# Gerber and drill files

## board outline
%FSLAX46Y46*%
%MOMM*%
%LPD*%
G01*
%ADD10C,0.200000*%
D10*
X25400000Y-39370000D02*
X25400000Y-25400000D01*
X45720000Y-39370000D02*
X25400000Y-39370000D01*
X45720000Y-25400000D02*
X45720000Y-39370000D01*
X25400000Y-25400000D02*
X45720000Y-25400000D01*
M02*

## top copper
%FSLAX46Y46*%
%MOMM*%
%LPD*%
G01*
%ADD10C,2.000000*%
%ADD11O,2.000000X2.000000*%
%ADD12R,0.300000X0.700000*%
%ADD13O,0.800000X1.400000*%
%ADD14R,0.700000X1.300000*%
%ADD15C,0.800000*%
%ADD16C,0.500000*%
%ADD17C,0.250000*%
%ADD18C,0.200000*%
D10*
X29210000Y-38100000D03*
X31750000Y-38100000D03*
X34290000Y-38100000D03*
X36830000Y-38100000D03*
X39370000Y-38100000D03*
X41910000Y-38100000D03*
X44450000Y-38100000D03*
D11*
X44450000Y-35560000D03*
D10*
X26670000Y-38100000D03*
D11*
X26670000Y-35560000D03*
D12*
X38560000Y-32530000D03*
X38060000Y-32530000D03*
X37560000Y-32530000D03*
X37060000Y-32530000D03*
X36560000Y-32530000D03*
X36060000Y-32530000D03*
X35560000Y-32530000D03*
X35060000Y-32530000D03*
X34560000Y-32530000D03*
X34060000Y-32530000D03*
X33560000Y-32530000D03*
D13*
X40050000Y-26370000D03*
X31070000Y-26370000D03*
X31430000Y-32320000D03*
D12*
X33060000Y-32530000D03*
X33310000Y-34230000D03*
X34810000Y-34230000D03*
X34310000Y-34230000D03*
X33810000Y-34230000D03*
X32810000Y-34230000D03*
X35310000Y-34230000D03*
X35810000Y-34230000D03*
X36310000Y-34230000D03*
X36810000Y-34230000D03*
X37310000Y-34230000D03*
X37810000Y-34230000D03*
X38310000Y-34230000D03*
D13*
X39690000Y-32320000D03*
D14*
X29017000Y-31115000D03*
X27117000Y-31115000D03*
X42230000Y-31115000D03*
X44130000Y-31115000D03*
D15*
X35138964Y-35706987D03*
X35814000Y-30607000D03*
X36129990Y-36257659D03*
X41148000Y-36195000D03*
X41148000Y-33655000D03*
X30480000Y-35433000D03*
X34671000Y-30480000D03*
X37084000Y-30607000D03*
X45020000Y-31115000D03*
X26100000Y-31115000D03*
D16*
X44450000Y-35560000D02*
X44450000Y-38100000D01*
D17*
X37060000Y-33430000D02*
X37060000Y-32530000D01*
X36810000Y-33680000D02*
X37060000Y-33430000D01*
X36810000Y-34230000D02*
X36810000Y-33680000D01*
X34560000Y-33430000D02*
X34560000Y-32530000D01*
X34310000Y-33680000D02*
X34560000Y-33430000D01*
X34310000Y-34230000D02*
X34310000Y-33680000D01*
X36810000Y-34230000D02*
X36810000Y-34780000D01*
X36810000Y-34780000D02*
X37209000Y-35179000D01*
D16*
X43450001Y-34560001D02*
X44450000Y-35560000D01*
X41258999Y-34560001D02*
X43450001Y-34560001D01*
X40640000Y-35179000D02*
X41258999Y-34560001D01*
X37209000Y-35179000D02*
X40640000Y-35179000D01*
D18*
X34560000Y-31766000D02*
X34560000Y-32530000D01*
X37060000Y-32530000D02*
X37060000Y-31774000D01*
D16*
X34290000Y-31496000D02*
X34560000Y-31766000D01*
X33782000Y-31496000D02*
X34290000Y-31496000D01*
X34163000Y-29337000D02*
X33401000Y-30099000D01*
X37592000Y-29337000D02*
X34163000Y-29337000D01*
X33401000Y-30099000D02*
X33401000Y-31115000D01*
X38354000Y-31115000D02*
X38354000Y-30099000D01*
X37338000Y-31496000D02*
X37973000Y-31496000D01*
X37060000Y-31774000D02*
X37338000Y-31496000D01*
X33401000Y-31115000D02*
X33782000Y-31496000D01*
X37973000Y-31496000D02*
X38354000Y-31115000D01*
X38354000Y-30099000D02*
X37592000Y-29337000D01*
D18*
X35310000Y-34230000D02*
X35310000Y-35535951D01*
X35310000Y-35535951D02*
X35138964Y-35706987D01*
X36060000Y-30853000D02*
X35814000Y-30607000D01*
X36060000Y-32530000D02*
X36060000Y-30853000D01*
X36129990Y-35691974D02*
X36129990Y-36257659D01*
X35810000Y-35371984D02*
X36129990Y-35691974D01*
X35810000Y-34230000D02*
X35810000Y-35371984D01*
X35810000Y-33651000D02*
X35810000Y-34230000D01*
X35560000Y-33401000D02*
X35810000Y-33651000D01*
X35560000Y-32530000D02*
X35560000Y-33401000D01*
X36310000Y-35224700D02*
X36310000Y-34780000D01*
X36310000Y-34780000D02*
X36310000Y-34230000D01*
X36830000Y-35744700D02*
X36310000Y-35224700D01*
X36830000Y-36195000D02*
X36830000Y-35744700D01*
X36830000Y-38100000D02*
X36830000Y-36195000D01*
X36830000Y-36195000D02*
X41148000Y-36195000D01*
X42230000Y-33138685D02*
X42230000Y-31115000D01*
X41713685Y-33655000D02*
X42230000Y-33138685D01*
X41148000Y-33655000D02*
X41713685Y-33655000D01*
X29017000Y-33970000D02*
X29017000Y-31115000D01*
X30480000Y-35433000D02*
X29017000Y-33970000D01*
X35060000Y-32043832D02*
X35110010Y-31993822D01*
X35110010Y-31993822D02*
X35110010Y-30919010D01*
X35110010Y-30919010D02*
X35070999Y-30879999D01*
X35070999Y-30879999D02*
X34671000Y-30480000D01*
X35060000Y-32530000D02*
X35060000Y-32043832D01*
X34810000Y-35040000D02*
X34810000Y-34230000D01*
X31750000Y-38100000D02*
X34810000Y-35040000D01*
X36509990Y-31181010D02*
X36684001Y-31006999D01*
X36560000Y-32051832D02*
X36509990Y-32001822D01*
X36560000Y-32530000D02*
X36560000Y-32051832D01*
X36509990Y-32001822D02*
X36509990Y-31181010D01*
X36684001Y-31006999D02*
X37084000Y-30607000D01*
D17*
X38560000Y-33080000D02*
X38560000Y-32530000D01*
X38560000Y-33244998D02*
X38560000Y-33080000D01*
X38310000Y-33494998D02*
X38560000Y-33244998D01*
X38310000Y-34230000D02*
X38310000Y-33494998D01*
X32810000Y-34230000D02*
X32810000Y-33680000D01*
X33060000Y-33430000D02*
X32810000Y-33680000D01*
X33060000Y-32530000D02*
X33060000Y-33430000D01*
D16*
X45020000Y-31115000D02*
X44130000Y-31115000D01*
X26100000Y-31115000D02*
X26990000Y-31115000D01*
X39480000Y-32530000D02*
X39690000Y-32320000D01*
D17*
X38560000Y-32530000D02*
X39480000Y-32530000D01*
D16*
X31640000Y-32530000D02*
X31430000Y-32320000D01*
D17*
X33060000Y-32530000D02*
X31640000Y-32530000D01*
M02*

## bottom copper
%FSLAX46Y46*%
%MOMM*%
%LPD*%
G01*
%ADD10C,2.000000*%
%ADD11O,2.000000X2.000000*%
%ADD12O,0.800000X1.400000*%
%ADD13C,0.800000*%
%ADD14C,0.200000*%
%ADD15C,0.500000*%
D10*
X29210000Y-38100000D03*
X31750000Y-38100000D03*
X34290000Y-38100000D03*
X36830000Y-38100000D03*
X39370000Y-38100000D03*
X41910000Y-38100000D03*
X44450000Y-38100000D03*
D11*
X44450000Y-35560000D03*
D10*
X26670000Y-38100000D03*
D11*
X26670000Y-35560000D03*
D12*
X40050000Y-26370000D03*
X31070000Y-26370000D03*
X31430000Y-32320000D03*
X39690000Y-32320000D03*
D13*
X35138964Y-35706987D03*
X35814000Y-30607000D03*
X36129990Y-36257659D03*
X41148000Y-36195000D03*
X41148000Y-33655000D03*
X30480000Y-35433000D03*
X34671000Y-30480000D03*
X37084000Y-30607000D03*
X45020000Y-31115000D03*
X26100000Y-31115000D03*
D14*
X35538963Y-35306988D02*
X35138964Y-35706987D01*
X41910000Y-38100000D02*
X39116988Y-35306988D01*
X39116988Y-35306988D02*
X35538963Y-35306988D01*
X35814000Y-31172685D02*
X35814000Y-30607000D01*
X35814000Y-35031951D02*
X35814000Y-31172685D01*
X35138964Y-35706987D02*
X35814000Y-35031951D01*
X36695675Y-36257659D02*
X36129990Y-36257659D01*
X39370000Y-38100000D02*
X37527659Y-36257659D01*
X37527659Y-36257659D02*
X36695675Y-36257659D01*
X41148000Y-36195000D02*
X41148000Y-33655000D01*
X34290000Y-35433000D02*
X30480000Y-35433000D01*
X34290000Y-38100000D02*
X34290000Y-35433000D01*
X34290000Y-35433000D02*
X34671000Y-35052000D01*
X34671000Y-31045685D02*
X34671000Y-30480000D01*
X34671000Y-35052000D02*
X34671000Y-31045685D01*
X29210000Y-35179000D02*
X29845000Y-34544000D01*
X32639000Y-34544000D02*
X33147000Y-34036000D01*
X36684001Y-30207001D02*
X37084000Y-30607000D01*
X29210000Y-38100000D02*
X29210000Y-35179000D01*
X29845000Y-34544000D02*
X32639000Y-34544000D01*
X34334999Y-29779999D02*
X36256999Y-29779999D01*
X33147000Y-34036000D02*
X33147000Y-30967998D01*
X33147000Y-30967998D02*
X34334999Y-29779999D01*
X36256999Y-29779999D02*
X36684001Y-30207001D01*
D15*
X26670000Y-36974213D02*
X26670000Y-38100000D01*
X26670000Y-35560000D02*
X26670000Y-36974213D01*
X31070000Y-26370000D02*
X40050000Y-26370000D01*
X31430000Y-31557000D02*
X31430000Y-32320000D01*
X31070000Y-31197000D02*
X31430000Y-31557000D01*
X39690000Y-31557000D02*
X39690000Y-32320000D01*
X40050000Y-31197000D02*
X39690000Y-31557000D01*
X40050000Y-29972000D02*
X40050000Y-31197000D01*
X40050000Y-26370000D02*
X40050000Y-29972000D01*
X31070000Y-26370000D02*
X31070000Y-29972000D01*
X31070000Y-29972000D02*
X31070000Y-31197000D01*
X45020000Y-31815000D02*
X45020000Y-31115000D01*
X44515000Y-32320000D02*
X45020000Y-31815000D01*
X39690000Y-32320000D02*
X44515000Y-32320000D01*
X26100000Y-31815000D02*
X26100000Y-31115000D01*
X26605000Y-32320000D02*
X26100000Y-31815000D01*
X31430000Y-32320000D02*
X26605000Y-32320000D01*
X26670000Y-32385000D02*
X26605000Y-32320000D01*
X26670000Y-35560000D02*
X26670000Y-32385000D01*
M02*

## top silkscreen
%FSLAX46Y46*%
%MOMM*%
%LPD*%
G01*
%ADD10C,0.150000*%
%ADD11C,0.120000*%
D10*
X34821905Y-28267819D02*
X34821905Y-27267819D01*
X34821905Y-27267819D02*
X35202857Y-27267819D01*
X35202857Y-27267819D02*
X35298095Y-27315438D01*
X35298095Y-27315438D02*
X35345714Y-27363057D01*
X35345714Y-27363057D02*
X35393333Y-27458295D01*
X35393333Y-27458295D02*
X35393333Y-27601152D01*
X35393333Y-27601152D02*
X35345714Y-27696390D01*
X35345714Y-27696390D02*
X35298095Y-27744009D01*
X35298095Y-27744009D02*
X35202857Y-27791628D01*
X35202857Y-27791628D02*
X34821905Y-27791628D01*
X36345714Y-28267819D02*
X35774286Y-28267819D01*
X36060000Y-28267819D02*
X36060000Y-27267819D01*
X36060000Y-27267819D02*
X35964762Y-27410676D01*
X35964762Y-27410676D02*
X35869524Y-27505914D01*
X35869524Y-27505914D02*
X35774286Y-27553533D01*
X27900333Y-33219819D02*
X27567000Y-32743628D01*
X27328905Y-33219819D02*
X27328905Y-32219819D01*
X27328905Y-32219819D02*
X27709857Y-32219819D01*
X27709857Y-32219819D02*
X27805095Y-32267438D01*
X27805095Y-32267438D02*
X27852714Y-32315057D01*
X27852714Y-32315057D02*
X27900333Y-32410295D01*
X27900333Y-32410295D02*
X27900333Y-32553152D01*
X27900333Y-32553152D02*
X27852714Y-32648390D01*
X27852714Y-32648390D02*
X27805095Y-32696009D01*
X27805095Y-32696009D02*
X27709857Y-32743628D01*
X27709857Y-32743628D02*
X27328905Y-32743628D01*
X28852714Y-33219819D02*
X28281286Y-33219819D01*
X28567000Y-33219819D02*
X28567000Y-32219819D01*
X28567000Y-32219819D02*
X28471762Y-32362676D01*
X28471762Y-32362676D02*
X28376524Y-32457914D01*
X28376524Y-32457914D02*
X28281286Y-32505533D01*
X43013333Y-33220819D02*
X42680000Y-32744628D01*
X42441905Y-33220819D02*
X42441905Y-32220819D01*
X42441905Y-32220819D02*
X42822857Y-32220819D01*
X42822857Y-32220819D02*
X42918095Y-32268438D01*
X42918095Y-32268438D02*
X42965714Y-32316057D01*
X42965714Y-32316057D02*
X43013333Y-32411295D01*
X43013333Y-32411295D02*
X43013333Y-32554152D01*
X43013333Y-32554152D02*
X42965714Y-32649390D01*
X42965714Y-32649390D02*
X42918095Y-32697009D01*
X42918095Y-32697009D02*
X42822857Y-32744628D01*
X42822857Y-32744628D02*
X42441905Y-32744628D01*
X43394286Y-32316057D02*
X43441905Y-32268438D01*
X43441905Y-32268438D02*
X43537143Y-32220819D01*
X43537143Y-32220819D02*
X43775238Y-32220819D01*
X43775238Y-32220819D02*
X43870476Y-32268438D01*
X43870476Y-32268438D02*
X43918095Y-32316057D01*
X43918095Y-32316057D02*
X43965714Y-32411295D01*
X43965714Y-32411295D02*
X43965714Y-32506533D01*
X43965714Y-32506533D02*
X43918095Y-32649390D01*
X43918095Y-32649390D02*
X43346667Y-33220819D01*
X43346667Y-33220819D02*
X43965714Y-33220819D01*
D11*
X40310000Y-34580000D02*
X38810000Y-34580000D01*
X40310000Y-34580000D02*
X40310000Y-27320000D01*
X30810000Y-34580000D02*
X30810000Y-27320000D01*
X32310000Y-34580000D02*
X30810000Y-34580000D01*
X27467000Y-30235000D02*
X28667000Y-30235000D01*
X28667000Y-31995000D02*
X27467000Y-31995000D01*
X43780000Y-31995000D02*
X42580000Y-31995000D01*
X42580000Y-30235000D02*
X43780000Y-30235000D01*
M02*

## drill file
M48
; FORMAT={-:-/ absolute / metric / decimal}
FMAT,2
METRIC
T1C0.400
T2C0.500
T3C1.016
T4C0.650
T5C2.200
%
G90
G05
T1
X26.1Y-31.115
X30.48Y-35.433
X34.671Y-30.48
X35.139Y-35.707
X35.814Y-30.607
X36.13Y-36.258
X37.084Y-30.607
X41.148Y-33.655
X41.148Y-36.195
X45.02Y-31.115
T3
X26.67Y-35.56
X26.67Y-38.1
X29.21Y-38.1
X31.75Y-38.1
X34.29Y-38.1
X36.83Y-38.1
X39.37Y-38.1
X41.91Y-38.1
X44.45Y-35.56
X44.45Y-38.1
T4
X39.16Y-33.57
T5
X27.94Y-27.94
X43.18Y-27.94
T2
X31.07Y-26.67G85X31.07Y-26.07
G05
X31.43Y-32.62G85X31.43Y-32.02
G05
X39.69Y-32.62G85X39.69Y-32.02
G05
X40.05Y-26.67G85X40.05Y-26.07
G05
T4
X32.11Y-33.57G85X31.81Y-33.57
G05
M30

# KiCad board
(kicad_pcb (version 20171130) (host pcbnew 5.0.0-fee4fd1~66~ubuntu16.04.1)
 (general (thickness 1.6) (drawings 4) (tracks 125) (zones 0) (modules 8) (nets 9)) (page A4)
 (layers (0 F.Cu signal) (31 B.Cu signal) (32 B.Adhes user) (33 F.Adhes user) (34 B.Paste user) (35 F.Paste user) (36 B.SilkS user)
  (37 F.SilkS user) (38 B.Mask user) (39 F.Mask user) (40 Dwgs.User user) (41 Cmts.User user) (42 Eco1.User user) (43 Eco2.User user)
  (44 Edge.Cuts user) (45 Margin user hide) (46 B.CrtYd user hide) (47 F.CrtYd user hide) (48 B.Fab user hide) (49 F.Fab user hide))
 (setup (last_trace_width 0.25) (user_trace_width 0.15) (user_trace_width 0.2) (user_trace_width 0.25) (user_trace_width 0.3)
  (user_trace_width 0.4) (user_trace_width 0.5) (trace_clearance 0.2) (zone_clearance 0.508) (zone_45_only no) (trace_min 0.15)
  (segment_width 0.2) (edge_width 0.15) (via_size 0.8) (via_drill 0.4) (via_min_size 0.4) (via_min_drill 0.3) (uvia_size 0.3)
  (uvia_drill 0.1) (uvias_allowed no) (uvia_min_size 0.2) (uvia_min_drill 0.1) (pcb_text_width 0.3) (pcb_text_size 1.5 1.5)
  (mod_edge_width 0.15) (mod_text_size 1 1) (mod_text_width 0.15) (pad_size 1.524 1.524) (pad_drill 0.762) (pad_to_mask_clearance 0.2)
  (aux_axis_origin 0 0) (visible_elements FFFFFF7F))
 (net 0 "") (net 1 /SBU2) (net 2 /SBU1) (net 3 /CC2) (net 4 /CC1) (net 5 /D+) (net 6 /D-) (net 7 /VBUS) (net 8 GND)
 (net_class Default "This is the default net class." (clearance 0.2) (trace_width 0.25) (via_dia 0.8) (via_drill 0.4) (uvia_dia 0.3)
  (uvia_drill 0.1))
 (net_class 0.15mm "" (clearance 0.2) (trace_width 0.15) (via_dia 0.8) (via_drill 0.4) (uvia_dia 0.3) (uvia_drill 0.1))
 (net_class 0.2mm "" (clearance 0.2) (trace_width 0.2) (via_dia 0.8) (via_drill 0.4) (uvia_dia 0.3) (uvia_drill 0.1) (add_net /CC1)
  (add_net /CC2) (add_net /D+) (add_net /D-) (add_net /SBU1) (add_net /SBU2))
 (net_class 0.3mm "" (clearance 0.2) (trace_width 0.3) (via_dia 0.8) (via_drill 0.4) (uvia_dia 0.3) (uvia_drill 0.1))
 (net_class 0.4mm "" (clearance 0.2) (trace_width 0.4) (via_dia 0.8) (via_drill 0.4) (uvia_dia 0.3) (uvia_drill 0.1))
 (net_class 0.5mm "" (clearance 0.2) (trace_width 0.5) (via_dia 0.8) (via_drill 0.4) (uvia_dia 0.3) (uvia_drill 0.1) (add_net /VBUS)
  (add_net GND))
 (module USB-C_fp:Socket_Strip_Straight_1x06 (layer B.Cu) (at 35.56 38.1 180)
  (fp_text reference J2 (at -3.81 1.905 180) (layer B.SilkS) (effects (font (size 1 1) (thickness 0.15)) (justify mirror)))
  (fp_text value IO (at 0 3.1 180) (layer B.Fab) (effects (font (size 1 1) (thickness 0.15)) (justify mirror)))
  (pad 6 thru_hole circle (at 6.35 0 180) (size 2 2) (drill 1.016) (layers *.Cu *.Mask B.SilkS) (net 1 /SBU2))
  (pad 5 thru_hole circle (at 3.81 0 180) (size 2 2) (drill 1.016) (layers *.Cu *.Mask B.SilkS) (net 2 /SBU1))
  (pad 4 thru_hole circle (at 1.27 0 180) (size 2 2) (drill 1.016) (layers *.Cu *.Mask B.SilkS) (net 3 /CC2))
  (pad 3 thru_hole circle (at -1.27 0 180) (size 2 2) (drill 1.016) (layers *.Cu *.Mask B.SilkS) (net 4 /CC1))
  (pad 2 thru_hole circle (at -3.81 0 180) (size 2 2) (drill 1.016) (layers *.Cu *.Mask B.SilkS) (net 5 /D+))
  (pad 1 thru_hole circle (at -6.35 0 180) (size 2 2) (drill 1.016) (layers *.Cu *.Mask B.SilkS) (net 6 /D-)))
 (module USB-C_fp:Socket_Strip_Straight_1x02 (layer B.Cu) (at 44.45 36.83 90)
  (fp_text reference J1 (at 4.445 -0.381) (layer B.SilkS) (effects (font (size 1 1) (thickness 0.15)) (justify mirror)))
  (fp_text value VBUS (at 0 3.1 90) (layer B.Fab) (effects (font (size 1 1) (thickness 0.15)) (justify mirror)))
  (pad 1 thru_hole circle (at -1.27 0 90) (size 2 2) (drill 1.016) (layers *.Cu *.Mask B.SilkS) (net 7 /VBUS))
  (pad 2 thru_hole oval (at 1.27 0 90) (size 2 2) (drill 1.016) (layers *.Cu *.Mask B.SilkS) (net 7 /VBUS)))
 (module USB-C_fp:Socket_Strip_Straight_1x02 (layer B.Cu) (at 26.67 36.83 90)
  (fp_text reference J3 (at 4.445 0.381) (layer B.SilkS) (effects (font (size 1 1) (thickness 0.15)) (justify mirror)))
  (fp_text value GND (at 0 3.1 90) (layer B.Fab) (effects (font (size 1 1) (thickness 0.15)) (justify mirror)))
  (pad 1 thru_hole circle (at -1.27 0 90) (size 2 2) (drill 1.016) (layers *.Cu *.Mask B.SilkS) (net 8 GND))
  (pad 2 thru_hole oval (at 1.27 0 90) (size 2 2) (drill 1.016) (layers *.Cu *.Mask B.SilkS) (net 8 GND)))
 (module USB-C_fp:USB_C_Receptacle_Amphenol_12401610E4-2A (layer F.Cu) (at 35.56 29.21 180)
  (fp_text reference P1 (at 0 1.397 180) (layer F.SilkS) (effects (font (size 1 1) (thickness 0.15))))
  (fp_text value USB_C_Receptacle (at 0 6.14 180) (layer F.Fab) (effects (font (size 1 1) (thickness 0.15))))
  (fp_line (start -4.75 -5.37) (end -3.25 -5.37) (layer F.SilkS) (width 0.12))
  (fp_line (start -4.75 -5.37) (end -4.75 1.89) (layer F.SilkS) (width 0.12))
  (fp_line (start 4.75 -5.37) (end 4.75 1.89) (layer F.SilkS) (width 0.12))
  (fp_line (start 3.25 -5.37) (end 4.75 -5.37) (layer F.SilkS) (width 0.12))
  (pad B12 smd rect (at -3 -3.32 180) (size 0.3 0.7) (layers F.Cu F.Paste F.Mask) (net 8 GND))
  (pad B11 smd rect (at -2.5 -3.32 180) (size 0.3 0.7) (layers F.Cu F.Paste F.Mask))
  (pad B10 smd rect (at -2 -3.32 180) (size 0.3 0.7) (layers F.Cu F.Paste F.Mask))
  (pad B9 smd rect (at -1.5 -3.32 180) (size 0.3 0.7) (layers F.Cu F.Paste F.Mask) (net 7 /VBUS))
  (pad B8 smd rect (at -1 -3.32 180) (size 0.3 0.7) (layers F.Cu F.Paste F.Mask) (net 1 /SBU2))
  (pad B7 smd rect (at -0.5 -3.32 180) (size 0.3 0.7) (layers F.Cu F.Paste F.Mask) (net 6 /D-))
  (pad B6 smd rect (at 0 -3.32 180) (size 0.3 0.7) (layers F.Cu F.Paste F.Mask) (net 5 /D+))
  (pad B5 smd rect (at 0.5 -3.32 180) (size 0.3 0.7) (layers F.Cu F.Paste F.Mask) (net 3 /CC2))
  (pad B4 smd rect (at 1 -3.32 180) (size 0.3 0.7) (layers F.Cu F.Paste F.Mask) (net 7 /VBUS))
  (pad B3 smd rect (at 1.5 -3.32 180) (size 0.3 0.7) (layers F.Cu F.Paste F.Mask))
  (pad B2 smd rect (at 2 -3.32 180) (size 0.3 0.7) (layers F.Cu F.Paste F.Mask))
  (pad "" np_thru_hole circle (at -3.6 -4.36 180) (size 0.65 0.65) (drill 0.65) (layers *.Cu *.Mask))
  (pad "" np_thru_hole oval (at 3.6 -4.36 180) (size 0.95 0.65) (drill oval 0.95 0.65) (layers *.Cu *.Mask))
  (pad S1 thru_hole oval (at -4.49 2.84 180) (size 0.8 1.4) (drill oval 0.5 1.1) (layers *.Cu *.Mask) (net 8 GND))
  (pad S1 thru_hole oval (at 4.49 2.84 180) (size 0.8 1.4) (drill oval 0.5 1.1) (layers *.Cu *.Mask) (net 8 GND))
  (pad S1 thru_hole oval (at 4.13 -3.11 180) (size 0.8 1.4) (drill oval 0.5 1.1) (layers *.Cu *.Mask) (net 8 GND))
  (pad B1 smd rect (at 2.5 -3.32 180) (size 0.3 0.7) (layers F.Cu F.Paste F.Mask) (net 8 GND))
  (pad A11 smd rect (at 2.25 -5.02 180) (size 0.3 0.7) (layers F.Cu F.Paste F.Mask))
  (pad A8 smd rect (at 0.75 -5.02 180) (size 0.3 0.7) (layers F.Cu F.Paste F.Mask) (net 2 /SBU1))
  (pad A9 smd rect (at 1.25 -5.02 180) (size 0.3 0.7) (layers F.Cu F.Paste F.Mask) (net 7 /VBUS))
  (pad A10 smd rect (at 1.75 -5.02 180) (size 0.3 0.7) (layers F.Cu F.Paste F.Mask))
  (pad A12 smd rect (at 2.75 -5.02 180) (size 0.3 0.7) (layers F.Cu F.Paste F.Mask) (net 8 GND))
  (pad A7 smd rect (at 0.25 -5.02 180) (size 0.3 0.7) (layers F.Cu F.Paste F.Mask) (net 6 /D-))
  (pad A6 smd rect (at -0.25 -5.02 180) (size 0.3 0.7) (layers F.Cu F.Paste F.Mask) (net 5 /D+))
  (pad A5 smd rect (at -0.75 -5.02 180) (size 0.3 0.7) (layers F.Cu F.Paste F.Mask) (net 4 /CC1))
  (pad A4 smd rect (at -1.25 -5.02 180) (size 0.3 0.7) (layers F.Cu F.Paste F.Mask) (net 7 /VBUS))
  (pad A3 smd rect (at -1.75 -5.02 180) (size 0.3 0.7) (layers F.Cu F.Paste F.Mask))
  (pad A2 smd rect (at -2.25 -5.02 180) (size 0.3 0.7) (layers F.Cu F.Paste F.Mask))
  (pad A1 smd rect (at -2.75 -5.02 180) (size 0.3 0.7) (layers F.Cu F.Paste F.Mask) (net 8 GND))
  (pad S1 thru_hole oval (at -4.13 -3.11 180) (size 0.8 1.4) (drill oval 0.5 1.1) (layers *.Cu *.Mask) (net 8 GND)))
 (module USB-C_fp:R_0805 (layer F.Cu) (at 28.067 31.115 180)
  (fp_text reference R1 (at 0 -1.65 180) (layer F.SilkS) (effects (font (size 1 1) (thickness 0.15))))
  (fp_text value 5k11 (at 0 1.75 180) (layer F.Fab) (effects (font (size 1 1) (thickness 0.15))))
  (fp_line (start 0.6 0.88) (end -0.6 0.88) (layer F.SilkS) (width 0.12))
  (fp_line (start -0.6 -0.88) (end 0.6 -0.88) (layer F.SilkS) (width 0.12))
  (pad 1 smd rect (at -0.95 0 180) (size 0.7 1.3) (layers F.Cu F.Paste F.Mask) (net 3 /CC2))
  (pad 2 smd rect (at 0.95 0 180) (size 0.7 1.3) (layers F.Cu F.Paste F.Mask) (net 8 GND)))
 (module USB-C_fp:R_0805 (layer F.Cu) (at 43.18 31.115)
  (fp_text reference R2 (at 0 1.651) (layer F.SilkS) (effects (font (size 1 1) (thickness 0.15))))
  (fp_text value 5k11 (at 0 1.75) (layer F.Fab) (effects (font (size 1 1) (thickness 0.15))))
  (fp_line (start 0.6 0.88) (end -0.6 0.88) (layer F.SilkS) (width 0.12))
  (fp_line (start -0.6 -0.88) (end 0.6 -0.88) (layer F.SilkS) (width 0.12))
  (pad 1 smd rect (at -0.95 0) (size 0.7 1.3) (layers F.Cu F.Paste F.Mask) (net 4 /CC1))
  (pad 2 smd rect (at 0.95 0) (size 0.7 1.3) (layers F.Cu F.Paste F.Mask) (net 8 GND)))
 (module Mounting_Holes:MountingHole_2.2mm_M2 (layer F.Cu) (at 43.18 27.94)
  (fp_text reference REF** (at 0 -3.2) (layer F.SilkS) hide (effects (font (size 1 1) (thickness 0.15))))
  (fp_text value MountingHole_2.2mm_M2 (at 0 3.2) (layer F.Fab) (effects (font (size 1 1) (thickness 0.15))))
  (pad 1 np_thru_hole circle (at 0 0) (size 2.2 2.2) (drill 2.2) (layers *.Cu *.Mask)))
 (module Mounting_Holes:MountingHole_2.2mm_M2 (layer F.Cu) (at 27.94 27.94)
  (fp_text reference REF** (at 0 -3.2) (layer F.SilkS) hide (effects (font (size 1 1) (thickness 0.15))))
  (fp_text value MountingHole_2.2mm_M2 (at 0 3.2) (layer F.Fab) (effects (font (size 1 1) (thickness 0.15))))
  (pad 1 np_thru_hole circle (at 0 0) (size 2.2 2.2) (drill 2.2) (layers *.Cu *.Mask)))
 (gr_line (start 25.4 39.37) (end 25.4 25.4) (layer Edge.Cuts) (width 0.2))
 (gr_line (start 45.72 39.37) (end 25.4 39.37) (layer Edge.Cuts) (width 0.2))
 (gr_line (start 45.72 25.4) (end 45.72 39.37) (layer Edge.Cuts) (width 0.2))
 (gr_line (start 25.4 25.4) (end 45.72 25.4) (layer Edge.Cuts) (width 0.2))
 (segment (start 44.45 35.56) (end 44.45 38.1) (width 0.5) (layer F.Cu) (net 7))
 (segment (start 37.06 33.43) (end 37.06 32.53) (width 0.25) (layer F.Cu) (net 7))
 (segment (start 36.81 33.68) (end 37.06 33.43) (width 0.25) (layer F.Cu) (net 7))
 (segment (start 36.81 34.23) (end 36.81 33.68) (width 0.25) (layer F.Cu) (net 7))
 (segment (start 34.56 33.43) (end 34.56 32.53) (width 0.25) (layer F.Cu) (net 7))
 (segment (start 34.31 33.68) (end 34.56 33.43) (width 0.25) (layer F.Cu) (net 7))
 (segment (start 34.31 34.23) (end 34.31 33.68) (width 0.25) (layer F.Cu) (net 7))
 (segment (start 36.81 34.23) (end 36.81 34.78) (width 0.25) (layer F.Cu) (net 7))
 (segment (start 36.81 34.78) (end 37.209 35.179) (width 0.25) (layer F.Cu) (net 7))
 (segment (start 43.450001 34.560001) (end 44.45 35.56) (width 0.5) (layer F.Cu) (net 7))
 (segment (start 41.258999 34.560001) (end 43.450001 34.560001) (width 0.5) (layer F.Cu) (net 7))
 (segment (start 40.64 35.179) (end 41.258999 34.560001) (width 0.5) (layer F.Cu) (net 7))
 (segment (start 37.209 35.179) (end 40.64 35.179) (width 0.5) (layer F.Cu) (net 7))
 (segment (start 34.56 31.766) (end 34.56 32.53) (width 0.2) (layer F.Cu) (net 7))
 (segment (start 37.06 32.53) (end 37.06 31.774) (width 0.2) (layer F.Cu) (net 7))
 (segment (start 34.29 31.496) (end 34.56 31.766) (width 0.5) (layer F.Cu) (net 7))
 (segment (start 33.782 31.496) (end 34.29 31.496) (width 0.5) (layer F.Cu) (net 7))
 (segment (start 34.163 29.337) (end 33.401 30.099) (width 0.5) (layer F.Cu) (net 7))
 (segment (start 37.592 29.337) (end 34.163 29.337) (width 0.5) (layer F.Cu) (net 7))
 (segment (start 33.401 30.099) (end 33.401 31.115) (width 0.5) (layer F.Cu) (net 7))
 (segment (start 38.354 31.115) (end 38.354 30.099) (width 0.5) (layer F.Cu) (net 7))
 (segment (start 37.338 31.496) (end 37.973 31.496) (width 0.5) (layer F.Cu) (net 7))
 (segment (start 37.06 31.774) (end 37.338 31.496) (width 0.5) (layer F.Cu) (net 7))
 (segment (start 33.401 31.115) (end 33.782 31.496) (width 0.5) (layer F.Cu) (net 7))
 (segment (start 37.973 31.496) (end 38.354 31.115) (width 0.5) (layer F.Cu) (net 7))
 (segment (start 38.354 30.099) (end 37.592 29.337) (width 0.5) (layer F.Cu) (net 7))
 (via (at 35.138964 35.706987) (size 0.8) (drill 0.4) (layers F.Cu B.Cu) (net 6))
 (segment (start 35.538963 35.306988) (end 35.138964 35.706987) (width 0.2) (layer B.Cu) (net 6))
 (segment (start 41.91 38.1) (end 39.116988 35.306988) (width 0.2) (layer B.Cu) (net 6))
 (segment (start 35.31 34.23) (end 35.31 35.535951) (width 0.2) (layer F.Cu) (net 6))
 (segment (start 39.116988 35.306988) (end 35.538963 35.306988) (width 0.2) (layer B.Cu) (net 6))
 (segment (start 35.31 35.535951) (end 35.138964 35.706987) (width 0.2) (layer F.Cu) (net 6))
 (segment (start 35.814 31.172685) (end 35.814 30.607) (width 0.2) (layer B.Cu) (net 6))
 (segment (start 36.06 30.853) (end 35.814 30.607) (width 0.2) (layer F.Cu) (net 6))
 (segment (start 36.06 32.53) (end 36.06 30.853) (width 0.2) (layer F.Cu) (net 6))
 (via (at 35.814 30.607) (size 0.8) (drill 0.4) (layers F.Cu B.Cu) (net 6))
 (segment (start 35.814 35.031951) (end 35.814 31.172685) (width 0.2) (layer B.Cu) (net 6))
 (segment (start 35.138964 35.706987) (end 35.814 35.031951) (width 0.2) (layer B.Cu) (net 6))
 (segment (start 36.695675 36.257659) (end 36.12999 36.257659) (width 0.2) (layer B.Cu) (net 5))
 (segment (start 39.37 38.1) (end 37.527659 36.257659) (width 0.2) (layer B.Cu) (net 5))
 (segment (start 37.527659 36.257659) (end 36.695675 36.257659) (width 0.2) (layer B.Cu) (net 5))
 (via (at 36.12999 36.257659) (size 0.8) (drill 0.4) (layers F.Cu B.Cu) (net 5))
 (segment (start 36.12999 35.691974) (end 36.12999 36.257659) (width 0.2) (layer F.Cu) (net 5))
 (segment (start 35.81 35.371984) (end 36.12999 35.691974) (width 0.2) (layer F.Cu) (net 5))
 (segment (start 35.81 34.23) (end 35.81 35.371984) (width 0.2) (layer F.Cu) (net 5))
 (segment (start 35.81 33.651) (end 35.81 34.23) (width 0.2) (layer F.Cu) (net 5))
 (segment (start 35.56 33.401) (end 35.81 33.651) (width 0.2) (layer F.Cu) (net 5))
 (segment (start 35.56 32.53) (end 35.56 33.401) (width 0.2) (layer F.Cu) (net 5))
 (segment (start 36.31 35.2247) (end 36.31 34.78) (width 0.2) (layer F.Cu) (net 4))
 (segment (start 36.31 34.78) (end 36.31 34.23) (width 0.2) (layer F.Cu) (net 4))
 (segment (start 36.83 35.7447) (end 36.31 35.2247) (width 0.2) (layer F.Cu) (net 4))
 (segment (start 36.83 36.195) (end 36.83 35.7447) (width 0.2) (layer F.Cu) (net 4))
 (segment (start 36.83 38.1) (end 36.83 36.195) (width 0.2) (layer F.Cu) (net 4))
 (via (at 41.148 36.195) (size 0.8) (drill 0.4) (layers F.Cu B.Cu) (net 4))
 (segment (start 36.83 36.195) (end 41.148 36.195) (width 0.2) (layer F.Cu) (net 4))
 (via (at 41.148 33.655) (size 0.8) (drill 0.4) (layers F.Cu B.Cu) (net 4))
 (segment (start 41.148 36.195) (end 41.148 33.655) (width 0.2) (layer B.Cu) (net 4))
 (segment (start 42.23 33.138685) (end 42.23 31.115) (width 0.2) (layer F.Cu) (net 4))
 (segment (start 41.713685 33.655) (end 42.23 33.138685) (width 0.2) (layer F.Cu) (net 4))
 (segment (start 41.148 33.655) (end 41.713685 33.655) (width 0.2) (layer F.Cu) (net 4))
 (via (at 30.48 35.433) (size 0.8) (drill 0.4) (layers F.Cu B.Cu) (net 3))
 (segment (start 34.29 35.433) (end 30.48 35.433) (width 0.2) (layer B.Cu) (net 3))
 (segment (start 34.29 38.1) (end 34.29 35.433) (width 0.2) (layer B.Cu) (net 3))
 (segment (start 29.017 33.97) (end 29.017 31.115) (width 0.2) (layer F.Cu) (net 3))
 (segment (start 30.48 35.433) (end 29.017 33.97) (width 0.2) (layer F.Cu) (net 3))
 (segment (start 34.29 35.433) (end 34.671 35.052) (width 0.2) (layer B.Cu) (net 3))
 (segment (start 34.671 31.045685) (end 34.671 30.48) (width 0.2) (layer B.Cu) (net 3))
 (via (at 34.671 30.48) (size 0.8) (drill 0.4) (layers F.Cu B.Cu) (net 3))
 (segment (start 34.671 35.052) (end 34.671 31.045685) (width 0.2) (layer B.Cu) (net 3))
 (segment (start 35.06 32.043832) (end 35.11001 31.993822) (width 0.2) (layer F.Cu) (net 3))
 (segment (start 35.11001 31.993822) (end 35.11001 30.91901) (width 0.2) (layer F.Cu) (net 3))
 (segment (start 35.11001 30.91901) (end 35.070999 30.879999) (width 0.2) (layer F.Cu) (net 3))
 (segment (start 35.070999 30.879999) (end 34.671 30.48) (width 0.2) (layer F.Cu) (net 3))
 (segment (start 35.06 32.53) (end 35.06 32.043832) (width 0.2) (layer F.Cu) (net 3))
 (segment (start 34.81 35.04) (end 34.81 34.23) (width 0.2) (layer F.Cu) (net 2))
 (segment (start 31.75 38.1) (end 34.81 35.04) (width 0.2) (layer F.Cu) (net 2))
 (via (at 37.084 30.607) (size 0.8) (drill 0.4) (layers F.Cu B.Cu) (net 1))
 (segment (start 29.21 35.179) (end 29.845 34.544) (width 0.2) (layer B.Cu) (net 1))
 (segment (start 32.639 34.544) (end 33.147 34.036) (width 0.2) (layer B.Cu) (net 1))
 (segment (start 36.684001 30.207001) (end 37.084 30.607) (width 0.2) (layer B.Cu) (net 1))
 (segment (start 29.21 38.1) (end 29.21 35.179) (width 0.2) (layer B.Cu) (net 1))
 (segment (start 29.845 34.544) (end 32.639 34.544) (width 0.2) (layer B.Cu) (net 1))
 (segment (start 34.334999 29.779999) (end 36.256999 29.779999) (width 0.2) (layer B.Cu) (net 1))
 (segment (start 33.147 34.036) (end 33.147 30.967998) (width 0.2) (layer B.Cu) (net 1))
 (segment (start 33.147 30.967998) (end 34.334999 29.779999) (width 0.2) (layer B.Cu) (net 1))
 (segment (start 36.256999 29.779999) (end 36.684001 30.207001) (width 0.2) (layer B.Cu) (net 1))
 (segment (start 36.50999 31.18101) (end 36.684001 31.006999) (width 0.2) (layer F.Cu) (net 1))
 (segment (start 36.56 32.051832) (end 36.50999 32.001822) (width 0.2) (layer F.Cu) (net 1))
 (segment (start 36.56 32.53) (end 36.56 32.051832) (width 0.2) (layer F.Cu) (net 1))
 (segment (start 36.50999 32.001822) (end 36.50999 31.18101) (width 0.2) (layer F.Cu) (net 1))
 (segment (start 36.684001 31.006999) (end 37.084 30.607) (width 0.2) (layer F.Cu) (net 1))
 (segment (start 38.56 33.08) (end 38.56 32.53) (width 0.25) (layer F.Cu) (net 8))
 (segment (start 38.56 33.244998) (end 38.56 33.08) (width 0.25) (layer F.Cu) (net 8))
 (segment (start 38.31 33.494998) (end 38.56 33.244998) (width 0.25) (layer F.Cu) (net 8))
 (segment (start 38.31 34.23) (end 38.31 33.494998) (width 0.25) (layer F.Cu) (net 8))
 (segment (start 32.81 34.23) (end 32.81 33.68) (width 0.25) (layer F.Cu) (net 8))
 (segment (start 33.06 33.43) (end 32.81 33.68) (width 0.25) (layer F.Cu) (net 8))
 (segment (start 33.06 32.53) (end 33.06 33.43) (width 0.25) (layer F.Cu) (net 8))
 (segment (start 26.67 36.974213) (end 26.67 38.1) (width 0.5) (layer B.Cu) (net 8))
 (segment (start 26.67 35.56) (end 26.67 36.974213) (width 0.5) (layer B.Cu) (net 8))
 (segment (start 31.07 26.37) (end 40.05 26.37) (width 0.5) (layer B.Cu) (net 8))
 (via (at 45.02 31.115) (size 0.8) (drill 0.4) (layers F.Cu B.Cu) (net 8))
 (segment (start 45.02 31.115) (end 44.13 31.115) (width 0.5) (layer F.Cu) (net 8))
 (segment (start 31.43 31.557) (end 31.43 32.32) (width 0.5) (layer B.Cu) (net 8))
 (segment (start 31.07 31.197) (end 31.43 31.557) (width 0.5) (layer B.Cu) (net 8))
 (segment (start 39.69 31.557) (end 39.69 32.32) (width 0.5) (layer B.Cu) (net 8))
 (segment (start 40.05 31.197) (end 39.69 31.557) (width 0.5) (layer B.Cu) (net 8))
 (segment (start 40.05 29.972) (end 40.05 31.197) (width 0.5) (layer B.Cu) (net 8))
 (segment (start 40.05 26.37) (end 40.05 29.972) (width 0.5) (layer B.Cu) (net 8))
 (segment (start 31.07 26.37) (end 31.07 29.972) (width 0.5) (layer B.Cu) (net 8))
 (segment (start 31.07 29.972) (end 31.07 31.197) (width 0.5) (layer B.Cu) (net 8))
 (via (at 26.1 31.115) (size 0.8) (drill 0.4) (layers F.Cu B.Cu) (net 8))
 (segment (start 26.1 31.115) (end 26.99 31.115) (width 0.5) (layer F.Cu) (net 8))
 (segment (start 39.48 32.53) (end 39.69 32.32) (width 0.5) (layer F.Cu) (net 8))
 (segment (start 38.56 32.53) (end 39.48 32.53) (width 0.25) (layer F.Cu) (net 8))
 (segment (start 31.64 32.53) (end 31.43 32.32) (width 0.5) (layer F.Cu) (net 8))
 (segment (start 33.06 32.53) (end 31.64 32.53) (width 0.25) (layer F.Cu) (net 8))
 (segment (start 45.02 31.815) (end 45.02 31.115) (width 0.5) (layer B.Cu) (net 8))
 (segment (start 44.515 32.32) (end 45.02 31.815) (width 0.5) (layer B.Cu) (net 8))
 (segment (start 39.69 32.32) (end 44.515 32.32) (width 0.5) (layer B.Cu) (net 8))
 (segment (start 26.1 31.815) (end 26.1 31.115) (width 0.5) (layer B.Cu) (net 8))
 (segment (start 26.605 32.32) (end 26.1 31.815) (width 0.5) (layer B.Cu) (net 8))
 (segment (start 31.43 32.32) (end 26.605 32.32) (width 0.5) (layer B.Cu) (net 8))
 (segment (start 26.67 32.385) (end 26.605 32.32) (width 0.5) (layer B.Cu) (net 8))
 (segment (start 26.67 35.56) (end 26.67 32.385) (width 0.5) (layer B.Cu) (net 8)))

